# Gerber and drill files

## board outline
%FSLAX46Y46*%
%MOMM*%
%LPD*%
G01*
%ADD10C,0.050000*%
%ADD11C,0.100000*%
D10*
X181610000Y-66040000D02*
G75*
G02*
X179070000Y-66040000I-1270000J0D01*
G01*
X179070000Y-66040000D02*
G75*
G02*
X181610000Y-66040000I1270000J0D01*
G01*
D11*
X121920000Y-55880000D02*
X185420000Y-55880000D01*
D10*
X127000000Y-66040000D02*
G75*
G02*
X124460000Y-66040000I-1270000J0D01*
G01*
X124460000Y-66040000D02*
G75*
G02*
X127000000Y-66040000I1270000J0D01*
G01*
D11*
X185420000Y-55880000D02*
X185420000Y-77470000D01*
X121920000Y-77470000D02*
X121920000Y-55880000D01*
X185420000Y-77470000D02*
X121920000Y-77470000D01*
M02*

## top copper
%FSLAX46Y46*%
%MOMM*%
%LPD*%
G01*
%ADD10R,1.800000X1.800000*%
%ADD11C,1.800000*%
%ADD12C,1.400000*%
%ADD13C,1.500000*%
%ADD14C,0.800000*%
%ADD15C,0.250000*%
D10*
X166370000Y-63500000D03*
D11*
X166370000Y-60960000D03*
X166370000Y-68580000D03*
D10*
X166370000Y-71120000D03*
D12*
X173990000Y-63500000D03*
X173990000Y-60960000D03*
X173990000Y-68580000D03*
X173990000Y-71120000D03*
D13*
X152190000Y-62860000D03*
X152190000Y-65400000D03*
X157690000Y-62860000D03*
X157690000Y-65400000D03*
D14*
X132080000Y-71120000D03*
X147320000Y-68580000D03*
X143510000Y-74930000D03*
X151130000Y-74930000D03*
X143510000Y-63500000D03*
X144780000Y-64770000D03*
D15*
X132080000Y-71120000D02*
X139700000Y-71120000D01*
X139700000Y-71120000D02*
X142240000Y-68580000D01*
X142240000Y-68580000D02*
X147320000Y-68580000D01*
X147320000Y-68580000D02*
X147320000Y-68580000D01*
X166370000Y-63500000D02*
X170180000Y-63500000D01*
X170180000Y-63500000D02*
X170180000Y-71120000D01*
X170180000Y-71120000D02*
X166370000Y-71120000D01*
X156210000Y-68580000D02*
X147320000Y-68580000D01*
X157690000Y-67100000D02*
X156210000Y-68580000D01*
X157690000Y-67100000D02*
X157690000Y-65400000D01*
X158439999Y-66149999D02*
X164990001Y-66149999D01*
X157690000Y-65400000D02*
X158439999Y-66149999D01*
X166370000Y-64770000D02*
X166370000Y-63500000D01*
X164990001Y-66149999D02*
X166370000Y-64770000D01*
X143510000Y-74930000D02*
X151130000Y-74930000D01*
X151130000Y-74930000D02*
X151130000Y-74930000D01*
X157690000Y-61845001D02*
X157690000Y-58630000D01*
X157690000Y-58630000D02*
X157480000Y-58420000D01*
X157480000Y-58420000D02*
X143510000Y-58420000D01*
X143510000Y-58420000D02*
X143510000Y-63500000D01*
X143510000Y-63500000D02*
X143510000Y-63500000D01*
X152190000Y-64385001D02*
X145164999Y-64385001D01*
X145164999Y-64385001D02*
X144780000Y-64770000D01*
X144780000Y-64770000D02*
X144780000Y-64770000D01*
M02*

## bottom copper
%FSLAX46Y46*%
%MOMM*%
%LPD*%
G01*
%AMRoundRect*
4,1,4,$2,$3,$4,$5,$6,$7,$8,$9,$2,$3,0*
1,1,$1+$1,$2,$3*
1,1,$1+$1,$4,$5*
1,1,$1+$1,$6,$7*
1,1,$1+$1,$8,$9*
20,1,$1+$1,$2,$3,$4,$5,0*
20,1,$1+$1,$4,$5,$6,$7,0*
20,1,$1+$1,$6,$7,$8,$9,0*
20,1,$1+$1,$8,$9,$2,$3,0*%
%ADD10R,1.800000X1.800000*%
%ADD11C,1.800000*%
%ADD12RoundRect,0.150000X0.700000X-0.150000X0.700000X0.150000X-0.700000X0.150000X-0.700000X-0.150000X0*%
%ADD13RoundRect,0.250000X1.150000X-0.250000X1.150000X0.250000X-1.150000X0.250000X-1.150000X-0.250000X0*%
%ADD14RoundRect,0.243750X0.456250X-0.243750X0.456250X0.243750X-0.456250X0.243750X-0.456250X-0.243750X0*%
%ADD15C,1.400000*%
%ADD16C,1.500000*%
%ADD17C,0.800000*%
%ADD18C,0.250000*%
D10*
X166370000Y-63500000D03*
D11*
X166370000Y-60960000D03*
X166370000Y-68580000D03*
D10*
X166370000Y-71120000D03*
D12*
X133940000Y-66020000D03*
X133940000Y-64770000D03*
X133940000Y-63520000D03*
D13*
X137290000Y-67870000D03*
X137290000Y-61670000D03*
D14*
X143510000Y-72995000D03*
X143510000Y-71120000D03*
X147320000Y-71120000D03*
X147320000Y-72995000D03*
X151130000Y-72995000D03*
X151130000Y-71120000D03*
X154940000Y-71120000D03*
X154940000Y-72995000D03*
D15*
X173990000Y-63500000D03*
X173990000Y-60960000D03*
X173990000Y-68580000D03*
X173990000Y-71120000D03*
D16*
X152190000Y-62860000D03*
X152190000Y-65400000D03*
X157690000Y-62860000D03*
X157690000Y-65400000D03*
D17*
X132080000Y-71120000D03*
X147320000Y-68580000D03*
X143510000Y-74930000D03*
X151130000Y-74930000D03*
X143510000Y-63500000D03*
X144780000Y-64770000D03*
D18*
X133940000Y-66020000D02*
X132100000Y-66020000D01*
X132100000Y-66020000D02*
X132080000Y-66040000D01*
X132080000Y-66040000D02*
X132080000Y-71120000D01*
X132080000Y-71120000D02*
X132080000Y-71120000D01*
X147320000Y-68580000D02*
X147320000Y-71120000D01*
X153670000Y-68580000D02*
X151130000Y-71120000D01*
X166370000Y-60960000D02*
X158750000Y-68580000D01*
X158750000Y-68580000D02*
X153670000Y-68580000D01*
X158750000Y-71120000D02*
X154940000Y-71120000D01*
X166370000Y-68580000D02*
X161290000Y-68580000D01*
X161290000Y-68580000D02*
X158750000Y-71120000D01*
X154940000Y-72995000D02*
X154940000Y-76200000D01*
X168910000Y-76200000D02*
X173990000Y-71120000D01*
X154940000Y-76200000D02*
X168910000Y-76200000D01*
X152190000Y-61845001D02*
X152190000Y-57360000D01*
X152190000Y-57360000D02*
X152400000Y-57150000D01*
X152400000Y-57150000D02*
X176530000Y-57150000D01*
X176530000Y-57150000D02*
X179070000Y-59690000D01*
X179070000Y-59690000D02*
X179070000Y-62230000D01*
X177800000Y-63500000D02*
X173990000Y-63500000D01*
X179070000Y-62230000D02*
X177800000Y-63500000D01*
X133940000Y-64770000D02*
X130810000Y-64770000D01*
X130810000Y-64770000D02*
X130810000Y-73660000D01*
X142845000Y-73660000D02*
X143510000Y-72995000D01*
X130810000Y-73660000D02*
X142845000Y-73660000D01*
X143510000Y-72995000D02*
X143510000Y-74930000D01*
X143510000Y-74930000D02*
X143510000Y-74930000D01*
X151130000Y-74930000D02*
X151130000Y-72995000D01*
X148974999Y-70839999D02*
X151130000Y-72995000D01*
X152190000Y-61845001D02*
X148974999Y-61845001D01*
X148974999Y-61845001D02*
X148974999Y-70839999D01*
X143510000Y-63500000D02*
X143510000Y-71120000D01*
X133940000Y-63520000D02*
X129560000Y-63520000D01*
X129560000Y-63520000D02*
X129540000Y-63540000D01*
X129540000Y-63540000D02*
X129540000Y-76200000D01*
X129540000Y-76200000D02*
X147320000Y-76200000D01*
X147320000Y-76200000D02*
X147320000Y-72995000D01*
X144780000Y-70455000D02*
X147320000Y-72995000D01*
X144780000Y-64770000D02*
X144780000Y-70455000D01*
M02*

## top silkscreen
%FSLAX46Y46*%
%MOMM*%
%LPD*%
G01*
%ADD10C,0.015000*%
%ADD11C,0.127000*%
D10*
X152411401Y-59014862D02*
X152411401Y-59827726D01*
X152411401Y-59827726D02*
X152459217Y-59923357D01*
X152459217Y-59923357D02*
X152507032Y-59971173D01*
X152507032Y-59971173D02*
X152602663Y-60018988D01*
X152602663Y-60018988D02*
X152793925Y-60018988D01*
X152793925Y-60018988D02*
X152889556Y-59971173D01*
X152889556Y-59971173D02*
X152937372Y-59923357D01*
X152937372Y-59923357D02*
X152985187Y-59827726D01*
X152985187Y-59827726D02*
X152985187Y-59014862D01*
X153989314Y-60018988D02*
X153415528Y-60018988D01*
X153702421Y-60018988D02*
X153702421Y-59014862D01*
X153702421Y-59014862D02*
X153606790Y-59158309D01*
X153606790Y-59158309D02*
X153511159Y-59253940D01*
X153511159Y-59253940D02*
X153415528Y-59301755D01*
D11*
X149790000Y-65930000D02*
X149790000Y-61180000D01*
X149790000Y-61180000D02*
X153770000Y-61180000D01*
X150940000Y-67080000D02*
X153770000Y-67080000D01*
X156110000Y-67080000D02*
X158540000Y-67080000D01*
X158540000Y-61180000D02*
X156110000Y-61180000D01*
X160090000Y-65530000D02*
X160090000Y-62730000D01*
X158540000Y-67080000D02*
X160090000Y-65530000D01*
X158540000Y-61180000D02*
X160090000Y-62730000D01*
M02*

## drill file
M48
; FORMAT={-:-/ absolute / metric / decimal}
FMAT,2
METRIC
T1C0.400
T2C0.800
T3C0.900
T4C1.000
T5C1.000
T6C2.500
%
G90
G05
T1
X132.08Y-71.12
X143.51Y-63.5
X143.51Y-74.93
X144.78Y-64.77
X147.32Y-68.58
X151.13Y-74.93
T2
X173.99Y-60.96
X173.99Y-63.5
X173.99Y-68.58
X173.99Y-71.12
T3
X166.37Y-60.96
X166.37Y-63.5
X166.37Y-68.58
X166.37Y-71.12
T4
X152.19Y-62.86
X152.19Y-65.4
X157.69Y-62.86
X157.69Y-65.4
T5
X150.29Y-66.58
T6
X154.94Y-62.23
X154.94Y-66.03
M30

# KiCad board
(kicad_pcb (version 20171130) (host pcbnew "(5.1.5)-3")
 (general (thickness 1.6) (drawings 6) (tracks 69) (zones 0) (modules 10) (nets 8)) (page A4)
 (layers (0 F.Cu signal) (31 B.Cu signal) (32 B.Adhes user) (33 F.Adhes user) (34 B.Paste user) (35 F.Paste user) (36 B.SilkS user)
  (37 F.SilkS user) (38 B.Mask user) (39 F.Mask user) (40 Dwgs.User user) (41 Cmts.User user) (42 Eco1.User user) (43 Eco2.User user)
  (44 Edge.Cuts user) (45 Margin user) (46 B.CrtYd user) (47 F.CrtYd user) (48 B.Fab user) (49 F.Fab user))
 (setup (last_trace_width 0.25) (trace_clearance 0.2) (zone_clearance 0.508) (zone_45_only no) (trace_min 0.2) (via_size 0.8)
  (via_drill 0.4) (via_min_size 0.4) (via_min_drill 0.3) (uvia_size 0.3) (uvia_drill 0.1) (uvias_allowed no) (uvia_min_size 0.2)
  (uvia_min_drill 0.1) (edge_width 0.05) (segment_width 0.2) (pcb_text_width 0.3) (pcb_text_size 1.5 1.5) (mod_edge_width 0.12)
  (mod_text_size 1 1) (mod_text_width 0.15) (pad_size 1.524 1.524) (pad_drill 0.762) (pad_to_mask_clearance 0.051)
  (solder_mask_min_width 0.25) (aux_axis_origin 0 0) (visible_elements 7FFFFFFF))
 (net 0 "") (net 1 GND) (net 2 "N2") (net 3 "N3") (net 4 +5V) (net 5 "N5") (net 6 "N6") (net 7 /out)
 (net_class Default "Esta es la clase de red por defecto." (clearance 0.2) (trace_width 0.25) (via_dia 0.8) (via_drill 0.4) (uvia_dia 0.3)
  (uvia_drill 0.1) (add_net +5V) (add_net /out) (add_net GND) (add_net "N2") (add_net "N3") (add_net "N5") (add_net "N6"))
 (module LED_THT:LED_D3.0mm (layer B.Cu) (at 166.37 63.5 90)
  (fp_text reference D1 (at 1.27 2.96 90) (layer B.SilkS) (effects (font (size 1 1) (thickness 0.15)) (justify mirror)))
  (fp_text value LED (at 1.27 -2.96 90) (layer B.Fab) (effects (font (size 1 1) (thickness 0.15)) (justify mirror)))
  (pad 1 thru_hole rect (at 0 0 90) (size 1.8 1.8) (drill 0.9) (layers *.Cu *.Mask) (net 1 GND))
  (pad 2 thru_hole circle (at 2.54 0 90) (size 1.8 1.8) (drill 0.9) (layers *.Cu *.Mask) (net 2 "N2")))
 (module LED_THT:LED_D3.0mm (layer B.Cu) (at 166.37 71.12 90)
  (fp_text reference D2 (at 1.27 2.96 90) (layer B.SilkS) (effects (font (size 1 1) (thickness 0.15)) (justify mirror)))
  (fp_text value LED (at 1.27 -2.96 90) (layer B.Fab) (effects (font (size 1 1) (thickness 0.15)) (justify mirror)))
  (pad 2 thru_hole circle (at 2.54 0 90) (size 1.8 1.8) (drill 0.9) (layers *.Cu *.Mask) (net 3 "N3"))
  (pad 1 thru_hole rect (at 0 0 90) (size 1.8 1.8) (drill 0.9) (layers *.Cu *.Mask) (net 1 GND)))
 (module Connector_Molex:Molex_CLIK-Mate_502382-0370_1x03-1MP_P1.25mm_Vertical (layer B.Cu) (at 135.89 64.77 90)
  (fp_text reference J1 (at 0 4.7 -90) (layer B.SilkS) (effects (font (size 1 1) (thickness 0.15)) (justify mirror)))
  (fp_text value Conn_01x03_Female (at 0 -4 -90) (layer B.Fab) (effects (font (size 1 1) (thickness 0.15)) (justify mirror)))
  (pad 1 smd roundrect (at -1.25 -1.95 90) (size 0.6 1.7) (layers B.Cu B.Paste B.Mask) (roundrect_rratio 0.25) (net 1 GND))
  (pad 2 smd roundrect (at 0 -1.95 90) (size 0.6 1.7) (layers B.Cu B.Paste B.Mask) (roundrect_rratio 0.25) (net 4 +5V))
  (pad 3 smd roundrect (at 1.25 -1.95 90) (size 0.6 1.7) (layers B.Cu B.Paste B.Mask) (roundrect_rratio 0.25) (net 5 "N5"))
  (pad MP smd roundrect (at -3.1 1.4 90) (size 1 2.8) (layers B.Cu B.Paste B.Mask) (roundrect_rratio 0.25))
  (pad MP smd roundrect (at 3.1 1.4 90) (size 1 2.8) (layers B.Cu B.Paste B.Mask) (roundrect_rratio 0.25)))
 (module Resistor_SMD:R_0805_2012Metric (layer B.Cu) (at 143.51 72.0575 90)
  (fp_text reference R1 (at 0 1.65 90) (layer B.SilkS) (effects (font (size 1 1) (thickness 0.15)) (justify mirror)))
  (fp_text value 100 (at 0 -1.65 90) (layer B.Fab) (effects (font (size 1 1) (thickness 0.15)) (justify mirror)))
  (pad 1 smd roundrect (at -0.9375 0 90) (size 0.975 1.4) (layers B.Cu B.Paste B.Mask) (roundrect_rratio 0.25) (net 4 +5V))
  (pad 2 smd roundrect (at 0.9375 0 90) (size 0.975 1.4) (layers B.Cu B.Paste B.Mask) (roundrect_rratio 0.25) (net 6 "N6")))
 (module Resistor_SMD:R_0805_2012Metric (layer B.Cu) (at 147.32 72.0575 90)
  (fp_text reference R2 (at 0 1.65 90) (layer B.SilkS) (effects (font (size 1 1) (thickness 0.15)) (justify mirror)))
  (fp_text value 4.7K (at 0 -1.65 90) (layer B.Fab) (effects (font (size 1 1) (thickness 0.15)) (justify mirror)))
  (pad 2 smd roundrect (at 0.9375 0 90) (size 0.975 1.4) (layers B.Cu B.Paste B.Mask) (roundrect_rratio 0.25) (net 1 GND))
  (pad 1 smd roundrect (at -0.9375 0 90) (size 0.975 1.4) (layers B.Cu B.Paste B.Mask) (roundrect_rratio 0.25) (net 5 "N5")))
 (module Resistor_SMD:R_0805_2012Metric (layer B.Cu) (at 151.13 72.0575 90)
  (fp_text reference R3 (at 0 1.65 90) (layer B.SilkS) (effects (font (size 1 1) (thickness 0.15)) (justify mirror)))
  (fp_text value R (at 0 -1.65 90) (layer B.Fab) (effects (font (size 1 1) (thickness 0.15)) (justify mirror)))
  (pad 1 smd roundrect (at -0.9375 0 90) (size 0.975 1.4) (layers B.Cu B.Paste B.Mask) (roundrect_rratio 0.25) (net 4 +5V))
  (pad 2 smd roundrect (at 0.9375 0 90) (size 0.975 1.4) (layers B.Cu B.Paste B.Mask) (roundrect_rratio 0.25) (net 2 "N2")))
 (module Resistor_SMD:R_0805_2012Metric (layer B.Cu) (at 154.94 72.0575 90)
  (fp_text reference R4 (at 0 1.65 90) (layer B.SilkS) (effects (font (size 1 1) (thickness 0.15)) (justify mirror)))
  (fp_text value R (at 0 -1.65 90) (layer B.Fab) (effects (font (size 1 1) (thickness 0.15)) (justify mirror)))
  (pad 2 smd roundrect (at 0.9375 0 90) (size 0.975 1.4) (layers B.Cu B.Paste B.Mask) (roundrect_rratio 0.25) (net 3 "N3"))
  (pad 1 smd roundrect (at -0.9375 0 90) (size 0.975 1.4) (layers B.Cu B.Paste B.Mask) (roundrect_rratio 0.25) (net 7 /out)))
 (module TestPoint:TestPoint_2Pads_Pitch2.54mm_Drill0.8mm (layer B.Cu) (at 173.99 63.5 90)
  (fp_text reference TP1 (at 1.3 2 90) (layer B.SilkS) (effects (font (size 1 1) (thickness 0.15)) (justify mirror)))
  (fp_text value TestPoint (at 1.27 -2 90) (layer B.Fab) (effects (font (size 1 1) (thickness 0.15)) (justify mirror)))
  (pad 1 thru_hole circle (at 0 0 90) (size 1.4 1.4) (drill 0.8) (layers *.Cu *.Mask) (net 4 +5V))
  (pad 2 thru_hole circle (at 2.54 0 90) (size 1.4 1.4) (drill 0.8) (layers *.Cu *.Mask)))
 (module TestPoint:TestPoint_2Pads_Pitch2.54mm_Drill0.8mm (layer B.Cu) (at 173.99 71.12 90)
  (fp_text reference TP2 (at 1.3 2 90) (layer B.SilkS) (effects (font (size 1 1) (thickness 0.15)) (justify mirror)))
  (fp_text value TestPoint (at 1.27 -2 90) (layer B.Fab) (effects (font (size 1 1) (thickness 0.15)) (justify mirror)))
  (pad 2 thru_hole circle (at 2.54 0 90) (size 1.4 1.4) (drill 0.8) (layers *.Cu *.Mask))
  (pad 1 thru_hole circle (at 0 0 90) (size 1.4 1.4) (drill 0.8) (layers *.Cu *.Mask) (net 7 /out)))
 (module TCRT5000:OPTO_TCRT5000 (layer F.Cu) (at 154.94 64.13)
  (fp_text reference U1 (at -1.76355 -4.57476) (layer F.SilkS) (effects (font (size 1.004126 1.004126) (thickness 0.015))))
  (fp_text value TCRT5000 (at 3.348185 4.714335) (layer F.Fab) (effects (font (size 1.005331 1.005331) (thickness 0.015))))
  (fp_line (start -5.15 1.8) (end -5.15 -2.95) (layer F.SilkS) (width 0.127))
  (fp_line (start -5.15 -2.95) (end -1.17 -2.95) (layer F.SilkS) (width 0.127))
  (fp_line (start -4 2.95) (end -1.17 2.95) (layer F.SilkS) (width 0.127))
  (fp_line (start 1.17 2.95) (end 3.6 2.95) (layer F.SilkS) (width 0.127))
  (fp_line (start 3.6 -2.95) (end 1.17 -2.95) (layer F.SilkS) (width 0.127))
  (fp_line (start 5.15 1.4) (end 5.15 -1.4) (layer F.SilkS) (width 0.127))
  (fp_line (start 3.6 2.95) (end 5.15 1.4) (layer F.SilkS) (width 0.127))
  (fp_line (start 3.6 -2.95) (end 5.15 -1.4) (layer F.SilkS) (width 0.127))
  (pad COLL thru_hole circle (at -2.75 -1.27) (size 1.5 1.5) (drill 1) (layers *.Cu *.Mask) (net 4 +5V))
  (pad E thru_hole circle (at -2.75 1.27) (size 1.5 1.5) (drill 1) (layers *.Cu *.Mask) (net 5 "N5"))
  (pad A thru_hole circle (at 2.75 -1.27) (size 1.5 1.5) (drill 1) (layers *.Cu *.Mask) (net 6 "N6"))
  (pad CATH thru_hole circle (at 2.75 1.27) (size 1.5 1.5) (drill 1) (layers *.Cu *.Mask) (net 1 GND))
  (pad None np_thru_hole circle (at -4.65 2.45) (size 1 1) (drill 1) (layers *.Cu *.Mask))
  (pad None np_thru_hole circle (at 0 1.9) (size 2.5 2.5) (drill 2.5) (layers *.Cu *.Mask))
  (pad None np_thru_hole circle (at 0 -1.9) (size 2.5 2.5) (drill 2.5) (layers *.Cu *.Mask)))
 (gr_circle (center 180.34 66.04) (end 180.34 64.77) (layer Edge.Cuts) (width 0.05))
 (gr_line (start 121.92 55.88) (end 185.42 55.88) (layer Edge.Cuts) (width 0.1))
 (gr_circle (center 125.73 66.04) (end 125.73 64.77) (layer Edge.Cuts) (width 0.05))
 (gr_line (start 185.42 55.88) (end 185.42 77.47) (layer Edge.Cuts) (width 0.1))
 (gr_line (start 121.92 77.47) (end 121.92 55.88) (layer Edge.Cuts) (width 0.1))
 (gr_line (start 185.42 77.47) (end 121.92 77.47) (layer Edge.Cuts) (width 0.1))
 (segment (start 133.94 66.02) (end 132.1 66.02) (width 0.25) (layer B.Cu) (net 1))
 (segment (start 132.1 66.02) (end 132.08 66.04) (width 0.25) (layer B.Cu) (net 1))
 (segment (start 132.08 66.04) (end 132.08 71.12) (width 0.25) (layer B.Cu) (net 1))
 (segment (start 132.08 71.12) (end 132.08 71.12) (width 0.25) (layer B.Cu) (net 1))
 (via (at 132.08 71.12) (size 0.8) (drill 0.4) (layers F.Cu B.Cu) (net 1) (status 1000000))
 (segment (start 132.08 71.12) (end 139.7 71.12) (width 0.25) (layer F.Cu) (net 1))
 (segment (start 139.7 71.12) (end 142.24 68.58) (width 0.25) (layer F.Cu) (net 1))
 (segment (start 142.24 68.58) (end 147.32 68.58) (width 0.25) (layer F.Cu) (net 1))
 (segment (start 147.32 68.58) (end 147.32 68.58) (width 0.25) (layer F.Cu) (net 1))
 (via (at 147.32 68.58) (size 0.8) (drill 0.4) (layers F.Cu B.Cu) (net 1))
 (segment (start 147.32 68.58) (end 147.32 71.12) (width 0.25) (layer B.Cu) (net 1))
 (segment (start 166.37 63.5) (end 170.18 63.5) (width 0.25) (layer F.Cu) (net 1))
 (segment (start 170.18 63.5) (end 170.18 71.12) (width 0.25) (layer F.Cu) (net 1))
 (segment (start 170.18 71.12) (end 166.37 71.12) (width 0.25) (layer F.Cu) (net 1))
 (segment (start 156.21 68.58) (end 147.32 68.58) (width 0.25) (layer F.Cu) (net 1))
 (segment (start 157.69 67.1) (end 156.21 68.58) (width 0.25) (layer F.Cu) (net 1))
 (segment (start 157.69 67.1) (end 157.69 65.4) (width 0.25) (layer F.Cu) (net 1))
 (segment (start 158.439999 66.149999) (end 164.990001 66.149999) (width 0.25) (layer F.Cu) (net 1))
 (segment (start 157.69 65.4) (end 158.439999 66.149999) (width 0.25) (layer F.Cu) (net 1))
 (segment (start 166.37 64.77) (end 166.37 63.5) (width 0.25) (layer F.Cu) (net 1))
 (segment (start 164.990001 66.149999) (end 166.37 64.77) (width 0.25) (layer F.Cu) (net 1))
 (segment (start 153.67 68.58) (end 151.13 71.12) (width 0.25) (layer B.Cu) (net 2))
 (segment (start 166.37 60.96) (end 158.75 68.58) (width 0.25) (layer B.Cu) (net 2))
 (segment (start 158.75 68.58) (end 153.67 68.58) (width 0.25) (layer B.Cu) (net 2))
 (segment (start 158.75 71.12) (end 154.94 71.12) (width 0.25) (layer B.Cu) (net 3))
 (segment (start 166.37 68.58) (end 161.29 68.58) (width 0.25) (layer B.Cu) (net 3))
 (segment (start 161.29 68.58) (end 158.75 71.12) (width 0.25) (layer B.Cu) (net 3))
 (segment (start 154.94 72.995) (end 154.94 76.2) (width 0.25) (layer B.Cu) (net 7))
 (segment (start 168.91 76.2) (end 173.99 71.12) (width 0.25) (layer B.Cu) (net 7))
 (segment (start 154.94 76.2) (end 168.91 76.2) (width 0.25) (layer B.Cu) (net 7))
 (segment (start 152.19 61.845001) (end 152.19 57.36) (width 0.25) (layer B.Cu) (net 4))
 (segment (start 152.19 57.36) (end 152.4 57.15) (width 0.25) (layer B.Cu) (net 4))
 (segment (start 152.4 57.15) (end 176.53 57.15) (width 0.25) (layer B.Cu) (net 4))
 (segment (start 176.53 57.15) (end 179.07 59.69) (width 0.25) (layer B.Cu) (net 4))
 (segment (start 179.07 59.69) (end 179.07 62.23) (width 0.25) (layer B.Cu) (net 4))
 (segment (start 177.8 63.5) (end 173.99 63.5) (width 0.25) (layer B.Cu) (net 4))
 (segment (start 179.07 62.23) (end 177.8 63.5) (width 0.25) (layer B.Cu) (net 4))
 (segment (start 133.94 64.77) (end 130.81 64.77) (width 0.25) (layer B.Cu) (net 4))
 (segment (start 130.81 64.77) (end 130.81 73.66) (width 0.25) (layer B.Cu) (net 4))
 (segment (start 142.845 73.66) (end 143.51 72.995) (width 0.25) (layer B.Cu) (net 4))
 (segment (start 130.81 73.66) (end 142.845 73.66) (width 0.25) (layer B.Cu) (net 4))
 (segment (start 143.51 72.995) (end 143.51 74.93) (width 0.25) (layer B.Cu) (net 4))
 (segment (start 143.51 74.93) (end 143.51 74.93) (width 0.25) (layer B.Cu) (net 4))
 (via (at 143.51 74.93) (size 0.8) (drill 0.4) (layers F.Cu B.Cu) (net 4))
 (segment (start 143.51 74.93) (end 151.13 74.93) (width 0.25) (layer F.Cu) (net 4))
 (segment (start 151.13 74.93) (end 151.13 74.93) (width 0.25) (layer F.Cu) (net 4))
 (via (at 151.13 74.93) (size 0.8) (drill 0.4) (layers F.Cu B.Cu) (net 4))
 (segment (start 151.13 74.93) (end 151.13 72.995) (width 0.25) (layer B.Cu) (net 4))
 (segment (start 148.974999 70.839999) (end 151.13 72.995) (width 0.25) (layer B.Cu) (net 4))
 (segment (start 152.19 61.845001) (end 148.974999 61.845001) (width 0.25) (layer B.Cu) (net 4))
 (segment (start 148.974999 61.845001) (end 148.974999 70.839999) (width 0.25) (layer B.Cu) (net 4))
 (segment (start 157.69 61.845001) (end 157.69 58.63) (width 0.25) (layer F.Cu) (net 6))
 (segment (start 157.69 58.63) (end 157.48 58.42) (width 0.25) (layer F.Cu) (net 6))
 (segment (start 157.48 58.42) (end 143.51 58.42) (width 0.25) (layer F.Cu) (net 6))
 (segment (start 143.51 58.42) (end 143.51 63.5) (width 0.25) (layer F.Cu) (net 6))
 (segment (start 143.51 63.5) (end 143.51 63.5) (width 0.25) (layer F.Cu) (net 6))
 (via (at 143.51 63.5) (size 0.8) (drill 0.4) (layers F.Cu B.Cu) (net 6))
 (segment (start 143.51 63.5) (end 143.51 71.12) (width 0.25) (layer B.Cu) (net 6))
 (segment (start 133.94 63.52) (end 129.56 63.52) (width 0.25) (layer B.Cu) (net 5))
 (segment (start 129.56 63.52) (end 129.54 63.54) (width 0.25) (layer B.Cu) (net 5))
 (segment (start 129.54 63.54) (end 129.54 76.2) (width 0.25) (layer B.Cu) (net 5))
 (segment (start 129.54 76.2) (end 147.32 76.2) (width 0.25) (layer B.Cu) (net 5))
 (segment (start 147.32 76.2) (end 147.32 72.995) (width 0.25) (layer B.Cu) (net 5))
 (segment (start 152.19 64.385001) (end 145.164999 64.385001) (width 0.25) (layer F.Cu) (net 5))
 (segment (start 145.164999 64.385001) (end 144.78 64.77) (width 0.25) (layer F.Cu) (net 5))
 (segment (start 144.78 64.77) (end 144.78 64.77) (width 0.25) (layer F.Cu) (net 5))
 (via (at 144.78 64.77) (size 0.8) (drill 0.4) (layers F.Cu B.Cu) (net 5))
 (segment (start 144.78 70.455) (end 147.32 72.995) (width 0.25) (layer B.Cu) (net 5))
 (segment (start 144.78 64.77) (end 144.78 70.455) (width 0.25) (layer B.Cu) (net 5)))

